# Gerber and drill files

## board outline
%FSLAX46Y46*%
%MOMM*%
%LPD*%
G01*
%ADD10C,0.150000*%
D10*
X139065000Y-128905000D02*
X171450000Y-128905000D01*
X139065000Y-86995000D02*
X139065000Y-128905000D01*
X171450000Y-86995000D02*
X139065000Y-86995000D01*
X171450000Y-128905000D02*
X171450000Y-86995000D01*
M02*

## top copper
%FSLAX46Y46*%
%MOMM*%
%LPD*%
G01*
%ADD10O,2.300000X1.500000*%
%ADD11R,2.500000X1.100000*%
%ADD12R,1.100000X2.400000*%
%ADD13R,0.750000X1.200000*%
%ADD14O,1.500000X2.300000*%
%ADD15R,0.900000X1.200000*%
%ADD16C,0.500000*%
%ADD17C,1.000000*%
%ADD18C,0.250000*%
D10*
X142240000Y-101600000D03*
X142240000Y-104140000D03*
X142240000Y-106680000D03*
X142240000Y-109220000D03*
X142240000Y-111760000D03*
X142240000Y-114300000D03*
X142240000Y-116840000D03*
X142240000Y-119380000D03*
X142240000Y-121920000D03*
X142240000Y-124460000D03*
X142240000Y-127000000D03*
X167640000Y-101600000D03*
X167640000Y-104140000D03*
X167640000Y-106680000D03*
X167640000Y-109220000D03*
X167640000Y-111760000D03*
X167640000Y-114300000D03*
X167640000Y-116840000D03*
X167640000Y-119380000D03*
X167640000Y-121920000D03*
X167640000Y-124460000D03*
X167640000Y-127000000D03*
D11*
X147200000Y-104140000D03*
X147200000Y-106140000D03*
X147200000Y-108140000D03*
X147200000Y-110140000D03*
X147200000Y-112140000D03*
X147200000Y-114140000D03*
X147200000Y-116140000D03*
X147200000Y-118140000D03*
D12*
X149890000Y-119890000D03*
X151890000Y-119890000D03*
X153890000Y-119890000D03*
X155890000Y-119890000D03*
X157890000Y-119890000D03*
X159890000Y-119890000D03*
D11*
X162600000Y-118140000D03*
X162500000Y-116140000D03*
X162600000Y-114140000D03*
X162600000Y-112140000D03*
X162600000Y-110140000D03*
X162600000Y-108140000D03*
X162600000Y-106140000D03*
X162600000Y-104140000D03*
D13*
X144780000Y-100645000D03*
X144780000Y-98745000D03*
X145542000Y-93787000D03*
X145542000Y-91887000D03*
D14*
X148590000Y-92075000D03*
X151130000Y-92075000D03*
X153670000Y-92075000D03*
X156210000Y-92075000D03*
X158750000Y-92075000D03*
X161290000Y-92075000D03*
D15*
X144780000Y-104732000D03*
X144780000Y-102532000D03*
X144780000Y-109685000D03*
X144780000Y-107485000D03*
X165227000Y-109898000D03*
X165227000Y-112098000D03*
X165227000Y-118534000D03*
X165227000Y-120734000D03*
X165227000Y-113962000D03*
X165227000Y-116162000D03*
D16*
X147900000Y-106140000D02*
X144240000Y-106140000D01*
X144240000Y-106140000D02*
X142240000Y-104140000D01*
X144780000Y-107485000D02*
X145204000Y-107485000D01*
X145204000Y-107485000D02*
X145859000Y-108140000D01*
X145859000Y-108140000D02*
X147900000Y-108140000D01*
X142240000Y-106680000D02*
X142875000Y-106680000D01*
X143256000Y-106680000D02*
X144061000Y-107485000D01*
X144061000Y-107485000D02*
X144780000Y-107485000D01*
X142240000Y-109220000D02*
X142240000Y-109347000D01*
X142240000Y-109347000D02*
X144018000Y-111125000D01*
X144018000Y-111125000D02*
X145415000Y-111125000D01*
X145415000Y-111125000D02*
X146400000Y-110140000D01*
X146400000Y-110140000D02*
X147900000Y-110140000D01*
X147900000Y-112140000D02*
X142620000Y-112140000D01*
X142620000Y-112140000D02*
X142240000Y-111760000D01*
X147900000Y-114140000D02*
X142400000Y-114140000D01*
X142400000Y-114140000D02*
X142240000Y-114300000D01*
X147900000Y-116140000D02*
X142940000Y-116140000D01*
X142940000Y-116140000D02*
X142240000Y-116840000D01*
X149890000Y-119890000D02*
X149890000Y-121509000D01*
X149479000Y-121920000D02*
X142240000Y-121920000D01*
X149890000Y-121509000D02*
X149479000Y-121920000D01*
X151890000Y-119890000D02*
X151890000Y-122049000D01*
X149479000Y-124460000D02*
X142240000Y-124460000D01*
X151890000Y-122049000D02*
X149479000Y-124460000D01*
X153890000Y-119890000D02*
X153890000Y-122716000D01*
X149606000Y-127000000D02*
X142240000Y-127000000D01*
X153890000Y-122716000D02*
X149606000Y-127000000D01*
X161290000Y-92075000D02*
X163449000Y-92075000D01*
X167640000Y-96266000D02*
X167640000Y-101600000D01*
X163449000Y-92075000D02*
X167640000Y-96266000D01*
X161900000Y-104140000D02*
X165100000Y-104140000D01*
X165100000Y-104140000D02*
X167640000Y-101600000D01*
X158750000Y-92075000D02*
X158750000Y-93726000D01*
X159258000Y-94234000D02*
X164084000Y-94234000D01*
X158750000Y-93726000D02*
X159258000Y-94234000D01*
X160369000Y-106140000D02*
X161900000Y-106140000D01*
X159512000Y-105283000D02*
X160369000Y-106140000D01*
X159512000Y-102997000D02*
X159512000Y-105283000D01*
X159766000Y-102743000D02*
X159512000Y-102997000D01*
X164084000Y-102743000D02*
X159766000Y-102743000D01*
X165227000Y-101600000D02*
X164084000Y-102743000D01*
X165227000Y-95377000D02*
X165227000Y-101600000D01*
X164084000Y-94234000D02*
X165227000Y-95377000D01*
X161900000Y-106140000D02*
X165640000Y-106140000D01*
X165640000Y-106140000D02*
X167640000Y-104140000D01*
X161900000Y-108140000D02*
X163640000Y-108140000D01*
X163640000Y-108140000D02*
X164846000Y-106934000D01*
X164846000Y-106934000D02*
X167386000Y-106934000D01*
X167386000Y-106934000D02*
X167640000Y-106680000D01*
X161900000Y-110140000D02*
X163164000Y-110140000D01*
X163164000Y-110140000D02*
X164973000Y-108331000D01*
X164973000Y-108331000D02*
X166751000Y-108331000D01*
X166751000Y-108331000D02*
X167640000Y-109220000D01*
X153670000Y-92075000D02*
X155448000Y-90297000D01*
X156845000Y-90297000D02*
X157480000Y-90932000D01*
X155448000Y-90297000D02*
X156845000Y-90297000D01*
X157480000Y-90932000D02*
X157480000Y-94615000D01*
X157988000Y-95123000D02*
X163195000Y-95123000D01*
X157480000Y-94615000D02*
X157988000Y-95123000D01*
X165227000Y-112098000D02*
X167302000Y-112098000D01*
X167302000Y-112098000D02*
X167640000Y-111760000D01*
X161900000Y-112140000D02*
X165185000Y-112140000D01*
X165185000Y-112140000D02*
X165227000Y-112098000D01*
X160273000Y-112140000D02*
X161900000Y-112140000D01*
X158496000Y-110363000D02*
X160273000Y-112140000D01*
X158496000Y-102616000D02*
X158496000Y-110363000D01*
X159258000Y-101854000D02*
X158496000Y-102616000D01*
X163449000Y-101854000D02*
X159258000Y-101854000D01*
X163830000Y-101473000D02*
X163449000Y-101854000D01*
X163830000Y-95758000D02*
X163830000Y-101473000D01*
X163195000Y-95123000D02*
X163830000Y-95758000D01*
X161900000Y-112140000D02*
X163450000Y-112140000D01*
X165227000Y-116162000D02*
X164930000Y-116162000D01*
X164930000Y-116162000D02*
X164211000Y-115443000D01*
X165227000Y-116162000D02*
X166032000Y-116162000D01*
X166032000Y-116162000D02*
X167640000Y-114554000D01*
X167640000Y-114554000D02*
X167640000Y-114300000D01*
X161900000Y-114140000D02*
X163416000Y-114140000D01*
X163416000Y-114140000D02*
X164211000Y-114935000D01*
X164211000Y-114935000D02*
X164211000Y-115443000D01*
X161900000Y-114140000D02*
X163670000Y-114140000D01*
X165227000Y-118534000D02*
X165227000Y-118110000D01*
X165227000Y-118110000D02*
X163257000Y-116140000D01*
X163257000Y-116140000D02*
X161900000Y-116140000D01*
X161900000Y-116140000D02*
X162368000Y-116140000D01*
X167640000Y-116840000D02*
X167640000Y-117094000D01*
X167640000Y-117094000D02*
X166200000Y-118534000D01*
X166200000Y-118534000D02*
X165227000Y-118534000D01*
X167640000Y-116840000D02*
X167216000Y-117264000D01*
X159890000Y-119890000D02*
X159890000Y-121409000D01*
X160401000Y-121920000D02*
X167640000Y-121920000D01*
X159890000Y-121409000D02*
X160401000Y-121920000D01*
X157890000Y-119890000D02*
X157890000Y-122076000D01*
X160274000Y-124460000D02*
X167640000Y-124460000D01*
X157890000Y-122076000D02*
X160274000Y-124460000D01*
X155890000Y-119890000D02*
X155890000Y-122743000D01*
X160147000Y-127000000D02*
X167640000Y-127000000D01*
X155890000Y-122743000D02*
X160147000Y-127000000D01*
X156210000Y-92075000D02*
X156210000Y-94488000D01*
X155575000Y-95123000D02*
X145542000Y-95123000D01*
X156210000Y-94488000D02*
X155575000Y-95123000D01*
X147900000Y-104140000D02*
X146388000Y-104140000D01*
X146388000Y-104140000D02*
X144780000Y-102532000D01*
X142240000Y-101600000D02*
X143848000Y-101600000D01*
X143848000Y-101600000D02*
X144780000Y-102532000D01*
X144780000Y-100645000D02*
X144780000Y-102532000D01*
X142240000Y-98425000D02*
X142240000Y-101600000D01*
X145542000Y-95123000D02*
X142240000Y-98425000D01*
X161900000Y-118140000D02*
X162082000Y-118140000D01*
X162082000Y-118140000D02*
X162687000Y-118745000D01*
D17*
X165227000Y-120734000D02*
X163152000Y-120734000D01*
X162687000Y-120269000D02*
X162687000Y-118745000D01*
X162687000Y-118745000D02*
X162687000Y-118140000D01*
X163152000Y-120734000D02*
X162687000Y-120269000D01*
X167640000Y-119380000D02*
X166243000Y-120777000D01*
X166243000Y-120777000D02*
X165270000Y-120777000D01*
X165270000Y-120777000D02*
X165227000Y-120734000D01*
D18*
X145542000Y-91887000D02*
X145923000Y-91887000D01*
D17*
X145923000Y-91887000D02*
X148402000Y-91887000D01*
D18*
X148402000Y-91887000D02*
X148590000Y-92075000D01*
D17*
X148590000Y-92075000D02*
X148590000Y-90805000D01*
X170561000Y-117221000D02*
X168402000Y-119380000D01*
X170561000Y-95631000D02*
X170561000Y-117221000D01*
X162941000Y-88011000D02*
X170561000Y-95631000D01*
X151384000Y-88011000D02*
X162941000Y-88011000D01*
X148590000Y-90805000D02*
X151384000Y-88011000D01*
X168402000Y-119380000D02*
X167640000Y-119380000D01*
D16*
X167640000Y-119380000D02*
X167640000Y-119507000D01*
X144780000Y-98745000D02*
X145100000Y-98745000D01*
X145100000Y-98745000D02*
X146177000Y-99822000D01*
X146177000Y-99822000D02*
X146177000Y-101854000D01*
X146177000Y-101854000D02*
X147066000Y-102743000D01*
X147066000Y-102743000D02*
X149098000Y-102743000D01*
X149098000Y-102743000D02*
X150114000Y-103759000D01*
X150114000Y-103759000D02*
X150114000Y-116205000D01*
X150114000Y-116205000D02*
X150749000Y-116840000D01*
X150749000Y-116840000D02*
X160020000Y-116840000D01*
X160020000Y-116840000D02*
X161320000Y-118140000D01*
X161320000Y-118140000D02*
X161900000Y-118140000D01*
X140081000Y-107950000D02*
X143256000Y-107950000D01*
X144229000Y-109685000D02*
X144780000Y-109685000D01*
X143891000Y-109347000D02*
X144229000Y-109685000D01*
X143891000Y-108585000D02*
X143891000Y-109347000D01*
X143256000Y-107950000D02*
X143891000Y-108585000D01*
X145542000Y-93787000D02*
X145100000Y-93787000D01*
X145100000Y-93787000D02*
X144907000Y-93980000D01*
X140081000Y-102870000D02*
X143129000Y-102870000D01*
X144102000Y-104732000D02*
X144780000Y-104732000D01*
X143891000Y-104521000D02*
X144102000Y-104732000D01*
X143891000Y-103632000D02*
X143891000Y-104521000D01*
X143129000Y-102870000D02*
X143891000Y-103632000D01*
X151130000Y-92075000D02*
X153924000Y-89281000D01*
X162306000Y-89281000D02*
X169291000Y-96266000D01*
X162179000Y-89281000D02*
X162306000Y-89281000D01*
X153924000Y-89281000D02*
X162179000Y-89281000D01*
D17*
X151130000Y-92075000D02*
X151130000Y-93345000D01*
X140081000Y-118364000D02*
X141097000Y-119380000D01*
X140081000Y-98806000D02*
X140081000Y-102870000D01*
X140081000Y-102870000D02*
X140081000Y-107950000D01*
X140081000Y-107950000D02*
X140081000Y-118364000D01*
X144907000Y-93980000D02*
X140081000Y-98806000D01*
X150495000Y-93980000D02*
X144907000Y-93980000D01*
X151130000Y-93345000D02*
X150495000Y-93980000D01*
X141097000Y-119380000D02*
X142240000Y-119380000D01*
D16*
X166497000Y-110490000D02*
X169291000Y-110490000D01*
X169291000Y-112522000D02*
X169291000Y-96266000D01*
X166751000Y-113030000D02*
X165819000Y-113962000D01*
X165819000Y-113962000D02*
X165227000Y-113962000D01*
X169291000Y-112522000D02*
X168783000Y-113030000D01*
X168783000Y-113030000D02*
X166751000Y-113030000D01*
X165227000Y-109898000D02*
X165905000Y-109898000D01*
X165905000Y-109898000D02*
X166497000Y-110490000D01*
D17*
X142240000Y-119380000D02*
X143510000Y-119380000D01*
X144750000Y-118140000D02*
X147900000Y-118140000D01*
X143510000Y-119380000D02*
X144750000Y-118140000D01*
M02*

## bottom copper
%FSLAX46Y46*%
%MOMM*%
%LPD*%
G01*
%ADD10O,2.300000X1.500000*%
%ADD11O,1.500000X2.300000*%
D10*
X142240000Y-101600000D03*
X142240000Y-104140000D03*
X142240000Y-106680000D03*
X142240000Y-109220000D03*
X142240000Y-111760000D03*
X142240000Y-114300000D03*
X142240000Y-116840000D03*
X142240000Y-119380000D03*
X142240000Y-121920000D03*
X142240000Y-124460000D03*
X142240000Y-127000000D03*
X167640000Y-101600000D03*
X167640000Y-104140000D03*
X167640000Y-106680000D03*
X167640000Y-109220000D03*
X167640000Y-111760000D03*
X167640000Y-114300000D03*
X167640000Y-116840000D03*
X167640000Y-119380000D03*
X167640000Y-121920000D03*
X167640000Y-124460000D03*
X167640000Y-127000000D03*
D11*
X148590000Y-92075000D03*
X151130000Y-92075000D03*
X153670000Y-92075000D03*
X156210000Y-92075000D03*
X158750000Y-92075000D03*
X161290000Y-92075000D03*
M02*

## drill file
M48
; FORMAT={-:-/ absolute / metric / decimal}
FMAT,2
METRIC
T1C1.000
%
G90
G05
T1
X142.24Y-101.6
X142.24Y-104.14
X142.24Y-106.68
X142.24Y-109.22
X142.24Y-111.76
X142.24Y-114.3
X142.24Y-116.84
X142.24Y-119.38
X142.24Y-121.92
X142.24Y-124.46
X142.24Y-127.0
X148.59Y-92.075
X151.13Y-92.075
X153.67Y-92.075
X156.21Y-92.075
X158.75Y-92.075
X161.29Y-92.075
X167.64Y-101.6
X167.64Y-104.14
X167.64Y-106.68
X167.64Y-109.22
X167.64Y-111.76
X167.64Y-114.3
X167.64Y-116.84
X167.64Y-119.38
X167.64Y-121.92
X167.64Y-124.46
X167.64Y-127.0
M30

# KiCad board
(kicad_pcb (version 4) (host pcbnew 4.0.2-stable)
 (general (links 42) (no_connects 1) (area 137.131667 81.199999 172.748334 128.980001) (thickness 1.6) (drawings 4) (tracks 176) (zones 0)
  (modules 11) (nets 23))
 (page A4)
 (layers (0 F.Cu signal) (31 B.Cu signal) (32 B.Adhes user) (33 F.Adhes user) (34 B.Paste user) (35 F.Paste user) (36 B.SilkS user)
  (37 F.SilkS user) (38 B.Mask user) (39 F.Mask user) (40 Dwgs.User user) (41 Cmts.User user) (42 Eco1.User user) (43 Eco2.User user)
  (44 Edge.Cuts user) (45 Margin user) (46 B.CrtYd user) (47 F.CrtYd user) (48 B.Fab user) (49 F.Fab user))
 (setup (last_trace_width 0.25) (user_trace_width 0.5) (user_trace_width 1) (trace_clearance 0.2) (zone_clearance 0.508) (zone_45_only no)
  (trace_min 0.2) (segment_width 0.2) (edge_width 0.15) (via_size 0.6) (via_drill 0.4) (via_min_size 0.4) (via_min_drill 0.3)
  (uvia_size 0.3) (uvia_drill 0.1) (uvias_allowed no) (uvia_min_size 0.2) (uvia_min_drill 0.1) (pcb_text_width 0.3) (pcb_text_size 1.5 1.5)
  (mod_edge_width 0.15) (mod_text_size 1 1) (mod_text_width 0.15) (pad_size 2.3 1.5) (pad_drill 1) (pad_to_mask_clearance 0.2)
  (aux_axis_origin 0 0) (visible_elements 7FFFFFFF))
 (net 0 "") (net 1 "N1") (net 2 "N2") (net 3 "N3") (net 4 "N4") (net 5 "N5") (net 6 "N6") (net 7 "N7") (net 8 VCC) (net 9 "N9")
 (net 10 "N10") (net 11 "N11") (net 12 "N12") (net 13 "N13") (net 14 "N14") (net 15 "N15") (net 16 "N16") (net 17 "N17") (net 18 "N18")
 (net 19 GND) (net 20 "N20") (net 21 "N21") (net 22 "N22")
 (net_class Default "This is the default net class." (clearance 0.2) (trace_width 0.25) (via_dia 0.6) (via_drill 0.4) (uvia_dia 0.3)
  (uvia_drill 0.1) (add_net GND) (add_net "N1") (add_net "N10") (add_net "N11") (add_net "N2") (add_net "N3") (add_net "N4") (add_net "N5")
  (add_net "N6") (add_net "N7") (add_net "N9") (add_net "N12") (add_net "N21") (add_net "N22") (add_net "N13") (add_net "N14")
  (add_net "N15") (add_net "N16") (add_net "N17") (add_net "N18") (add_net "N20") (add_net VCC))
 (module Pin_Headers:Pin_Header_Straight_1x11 (layer F.Cu) (at 142.24 101.6)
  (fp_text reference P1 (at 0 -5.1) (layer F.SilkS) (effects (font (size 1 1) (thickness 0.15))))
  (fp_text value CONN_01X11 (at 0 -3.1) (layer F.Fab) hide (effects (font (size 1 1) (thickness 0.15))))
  (pad 1 thru_hole oval (at 0 0) (size 2.3 1.5) (drill 1) (layers *.Cu *.Mask) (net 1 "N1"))
  (pad 2 thru_hole oval (at 0 2.54) (size 2.3 1.5) (drill 1) (layers *.Cu *.Mask) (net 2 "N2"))
  (pad 3 thru_hole oval (at 0 5.08) (size 2.3 1.5) (drill 1) (layers *.Cu *.Mask) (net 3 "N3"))
  (pad 4 thru_hole oval (at 0 7.62) (size 2.3 1.5) (drill 1) (layers *.Cu *.Mask) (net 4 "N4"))
  (pad 5 thru_hole oval (at 0 10.16) (size 2.3 1.5) (drill 1) (layers *.Cu *.Mask) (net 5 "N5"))
  (pad 6 thru_hole oval (at 0 12.7) (size 2.3 1.5) (drill 1) (layers *.Cu *.Mask) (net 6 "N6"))
  (pad 7 thru_hole oval (at 0 15.24) (size 2.3 1.5) (drill 1) (layers *.Cu *.Mask) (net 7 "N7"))
  (pad 8 thru_hole oval (at 0 17.78) (size 2.3 1.5) (drill 1) (layers *.Cu *.Mask) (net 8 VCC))
  (pad 9 thru_hole oval (at 0 20.32) (size 2.3 1.5) (drill 1) (layers *.Cu *.Mask) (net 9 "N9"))
  (pad 10 thru_hole oval (at 0 22.86) (size 2.3 1.5) (drill 1) (layers *.Cu *.Mask) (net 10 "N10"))
  (pad 11 thru_hole oval (at 0 25.4) (size 2.3 1.5) (drill 1) (layers *.Cu *.Mask) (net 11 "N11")))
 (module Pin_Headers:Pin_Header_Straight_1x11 (layer F.Cu) (at 167.64 101.6)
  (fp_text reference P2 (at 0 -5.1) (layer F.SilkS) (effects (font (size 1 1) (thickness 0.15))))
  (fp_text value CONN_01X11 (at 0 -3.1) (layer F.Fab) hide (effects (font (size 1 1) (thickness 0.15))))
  (pad 1 thru_hole oval (at 0 0) (size 2.3 1.5) (drill 1) (layers *.Cu *.Mask) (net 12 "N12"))
  (pad 2 thru_hole oval (at 0 2.54) (size 2.3 1.5) (drill 1) (layers *.Cu *.Mask) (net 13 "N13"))
  (pad 3 thru_hole oval (at 0 5.08) (size 2.3 1.5) (drill 1) (layers *.Cu *.Mask) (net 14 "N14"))
  (pad 4 thru_hole oval (at 0 7.62) (size 2.3 1.5) (drill 1) (layers *.Cu *.Mask) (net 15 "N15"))
  (pad 5 thru_hole oval (at 0 10.16) (size 2.3 1.5) (drill 1) (layers *.Cu *.Mask) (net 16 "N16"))
  (pad 6 thru_hole oval (at 0 12.7) (size 2.3 1.5) (drill 1) (layers *.Cu *.Mask) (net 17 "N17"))
  (pad 7 thru_hole oval (at 0 15.24) (size 2.3 1.5) (drill 1) (layers *.Cu *.Mask) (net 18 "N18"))
  (pad 8 thru_hole oval (at 0 17.78) (size 2.3 1.5) (drill 1) (layers *.Cu *.Mask) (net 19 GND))
  (pad 9 thru_hole oval (at 0 20.32) (size 2.3 1.5) (drill 1) (layers *.Cu *.Mask) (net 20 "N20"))
  (pad 10 thru_hole oval (at 0 22.86) (size 2.3 1.5) (drill 1) (layers *.Cu *.Mask) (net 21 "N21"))
  (pad 11 thru_hole oval (at 0 25.4) (size 2.3 1.5) (drill 1) (layers *.Cu *.Mask) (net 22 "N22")))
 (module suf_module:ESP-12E (layer F.Cu) (at 147.9 104.14)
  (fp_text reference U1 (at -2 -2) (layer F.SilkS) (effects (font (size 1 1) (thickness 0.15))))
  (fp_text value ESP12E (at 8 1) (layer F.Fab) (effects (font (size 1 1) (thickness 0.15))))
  (pad 1 smd rect (at 0 0) (size 2.5 1.1) (drill (offset -0.7 0)) (layers F.Cu F.Paste F.Mask) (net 1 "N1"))
  (pad 2 smd rect (at 0 2) (size 2.5 1.1) (drill (offset -0.7 0)) (layers F.Cu F.Paste F.Mask) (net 2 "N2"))
  (pad 3 smd rect (at 0 4) (size 2.5 1.1) (drill (offset -0.7 0)) (layers F.Cu F.Paste F.Mask) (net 3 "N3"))
  (pad 4 smd rect (at 0 6) (size 2.5 1.1) (drill (offset -0.7 0)) (layers F.Cu F.Paste F.Mask) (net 4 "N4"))
  (pad 5 smd rect (at 0 8) (size 2.5 1.1) (drill (offset -0.7 0)) (layers F.Cu F.Paste F.Mask) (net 5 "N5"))
  (pad 6 smd rect (at 0 10) (size 2.5 1.1) (drill (offset -0.7 0)) (layers F.Cu F.Paste F.Mask) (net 6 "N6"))
  (pad 7 smd rect (at 0 12) (size 2.5 1.1) (drill (offset -0.7 0)) (layers F.Cu F.Paste F.Mask) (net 7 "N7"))
  (pad 8 smd rect (at 0 14) (size 2.5 1.1) (drill (offset -0.7 0)) (layers F.Cu F.Paste F.Mask) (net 8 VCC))
  (pad 17 smd rect (at 1.99 15.75 90) (size 2.4 1.1) (layers F.Cu F.Paste F.Mask) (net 9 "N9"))
  (pad 18 smd rect (at 3.99 15.75 90) (size 2.4 1.1) (layers F.Cu F.Paste F.Mask) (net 10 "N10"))
  (pad 19 smd rect (at 5.99 15.75 90) (size 2.4 1.1) (layers F.Cu F.Paste F.Mask) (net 11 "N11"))
  (pad 20 smd rect (at 7.99 15.75 90) (size 2.4 1.1) (layers F.Cu F.Paste F.Mask) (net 22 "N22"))
  (pad 21 smd rect (at 9.99 15.75 90) (size 2.4 1.1) (layers F.Cu F.Paste F.Mask) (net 21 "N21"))
  (pad 22 smd rect (at 11.99 15.75 90) (size 2.4 1.1) (layers F.Cu F.Paste F.Mask) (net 20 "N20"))
  (pad 9 smd rect (at 14 14) (size 2.5 1.1) (drill (offset 0.7 0)) (layers F.Cu F.Paste F.Mask) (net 19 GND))
  (pad 10 smd rect (at 14 12) (size 2.5 1.1) (drill (offset 0.6 0)) (layers F.Cu F.Paste F.Mask) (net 18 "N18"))
  (pad 11 smd rect (at 14 10) (size 2.5 1.1) (drill (offset 0.7 0)) (layers F.Cu F.Paste F.Mask) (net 17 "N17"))
  (pad 12 smd rect (at 14 8) (size 2.5 1.1) (drill (offset 0.7 0)) (layers F.Cu F.Paste F.Mask) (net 16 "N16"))
  (pad 13 smd rect (at 14 6) (size 2.5 1.1) (drill (offset 0.7 0)) (layers F.Cu F.Paste F.Mask) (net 15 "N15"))
  (pad 14 smd rect (at 14 4) (size 2.5 1.1) (drill (offset 0.7 0)) (layers F.Cu F.Paste F.Mask) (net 14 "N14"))
  (pad 15 smd rect (at 14 2) (size 2.5 1.1) (drill (offset 0.7 0)) (layers F.Cu F.Paste F.Mask) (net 13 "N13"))
  (pad 16 smd rect (at 14 0) (size 2.5 1.1) (drill (offset 0.7 0)) (layers F.Cu F.Paste F.Mask) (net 12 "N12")))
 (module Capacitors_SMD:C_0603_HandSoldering (layer F.Cu) (at 144.78 99.695 90)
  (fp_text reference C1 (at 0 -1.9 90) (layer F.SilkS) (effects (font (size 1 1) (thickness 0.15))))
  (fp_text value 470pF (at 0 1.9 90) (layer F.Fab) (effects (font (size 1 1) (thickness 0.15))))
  (pad 1 smd rect (at -0.95 0 90) (size 1.2 0.75) (layers F.Cu F.Paste F.Mask) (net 1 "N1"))
  (pad 2 smd rect (at 0.95 0 90) (size 1.2 0.75) (layers F.Cu F.Paste F.Mask) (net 19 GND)))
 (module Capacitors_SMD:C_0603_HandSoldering (layer F.Cu) (at 145.542 92.837 90)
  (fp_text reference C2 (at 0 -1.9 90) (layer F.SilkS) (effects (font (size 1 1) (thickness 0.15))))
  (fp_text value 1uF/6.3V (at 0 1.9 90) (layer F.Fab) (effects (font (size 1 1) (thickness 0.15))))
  (pad 1 smd rect (at -0.95 0 90) (size 1.2 0.75) (layers F.Cu F.Paste F.Mask) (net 8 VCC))
  (pad 2 smd rect (at 0.95 0 90) (size 1.2 0.75) (layers F.Cu F.Paste F.Mask) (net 19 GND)))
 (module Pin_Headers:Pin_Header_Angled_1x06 (layer F.Cu) (at 148.59 92.075 90)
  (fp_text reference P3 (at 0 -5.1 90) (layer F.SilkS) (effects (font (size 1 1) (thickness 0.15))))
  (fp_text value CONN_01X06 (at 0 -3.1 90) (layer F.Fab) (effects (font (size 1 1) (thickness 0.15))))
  (pad 1 thru_hole oval (at 0 0 90) (size 2.3 1.5) (drill 1) (layers *.Cu *.Mask) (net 19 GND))
  (pad 2 thru_hole oval (at 0 2.54 90) (size 2.3 1.5) (drill 1) (layers *.Cu *.Mask) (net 8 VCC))
  (pad 3 thru_hole oval (at 0 5.08 90) (size 2.3 1.5) (drill 1) (layers *.Cu *.Mask) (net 16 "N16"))
  (pad 4 thru_hole oval (at 0 7.62 90) (size 2.3 1.5) (drill 1) (layers *.Cu *.Mask) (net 1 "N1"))
  (pad 5 thru_hole oval (at 0 10.16 90) (size 2.3 1.5) (drill 1) (layers *.Cu *.Mask) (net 13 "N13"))
  (pad 6 thru_hole oval (at 0 12.7 90) (size 2.3 1.5) (drill 1) (layers *.Cu *.Mask) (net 12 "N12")))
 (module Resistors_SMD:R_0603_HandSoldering (layer F.Cu) (at 144.78 103.632 90)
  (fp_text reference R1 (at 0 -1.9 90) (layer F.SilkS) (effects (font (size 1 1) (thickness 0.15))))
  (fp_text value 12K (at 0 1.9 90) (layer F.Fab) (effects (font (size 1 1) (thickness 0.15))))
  (pad 1 smd rect (at -1.1 0 90) (size 1.2 0.9) (layers F.Cu F.Paste F.Mask) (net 8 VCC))
  (pad 2 smd rect (at 1.1 0 90) (size 1.2 0.9) (layers F.Cu F.Paste F.Mask) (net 1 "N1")))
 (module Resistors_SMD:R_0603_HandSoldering (layer F.Cu) (at 144.78 108.585 90)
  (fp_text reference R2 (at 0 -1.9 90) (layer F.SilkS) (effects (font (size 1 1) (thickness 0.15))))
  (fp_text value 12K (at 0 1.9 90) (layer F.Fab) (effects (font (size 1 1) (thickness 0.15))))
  (pad 1 smd rect (at -1.1 0 90) (size 1.2 0.9) (layers F.Cu F.Paste F.Mask) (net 8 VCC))
  (pad 2 smd rect (at 1.1 0 90) (size 1.2 0.9) (layers F.Cu F.Paste F.Mask) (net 3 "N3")))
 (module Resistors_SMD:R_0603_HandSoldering (layer F.Cu) (at 165.227 110.998 270)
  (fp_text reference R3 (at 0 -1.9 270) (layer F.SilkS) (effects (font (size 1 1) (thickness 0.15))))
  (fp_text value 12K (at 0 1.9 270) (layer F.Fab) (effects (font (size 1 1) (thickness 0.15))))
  (pad 1 smd rect (at -1.1 0 270) (size 1.2 0.9) (layers F.Cu F.Paste F.Mask) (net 8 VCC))
  (pad 2 smd rect (at 1.1 0 270) (size 1.2 0.9) (layers F.Cu F.Paste F.Mask) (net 16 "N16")))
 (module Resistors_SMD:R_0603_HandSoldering (layer F.Cu) (at 165.227 119.634 270)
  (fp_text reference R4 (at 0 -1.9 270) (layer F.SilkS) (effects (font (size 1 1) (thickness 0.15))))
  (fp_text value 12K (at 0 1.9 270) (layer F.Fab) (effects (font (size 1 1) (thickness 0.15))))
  (pad 1 smd rect (at -1.1 0 270) (size 1.2 0.9) (layers F.Cu F.Paste F.Mask) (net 18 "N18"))
  (pad 2 smd rect (at 1.1 0 270) (size 1.2 0.9) (layers F.Cu F.Paste F.Mask) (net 19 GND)))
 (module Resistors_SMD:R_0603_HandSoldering (layer F.Cu) (at 165.227 115.062 270)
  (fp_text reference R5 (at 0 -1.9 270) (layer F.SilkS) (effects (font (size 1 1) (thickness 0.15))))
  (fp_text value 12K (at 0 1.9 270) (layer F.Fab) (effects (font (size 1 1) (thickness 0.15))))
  (pad 1 smd rect (at -1.1 0 270) (size 1.2 0.9) (layers F.Cu F.Paste F.Mask) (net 8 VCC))
  (pad 2 smd rect (at 1.1 0 270) (size 1.2 0.9) (layers F.Cu F.Paste F.Mask) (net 17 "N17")))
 (gr_line (start 139.065 128.905) (end 171.45 128.905) (angle 90) (layer Edge.Cuts) (width 0.15))
 (gr_line (start 139.065 86.995) (end 139.065 128.905) (angle 90) (layer Edge.Cuts) (width 0.15))
 (gr_line (start 171.45 86.995) (end 139.065 86.995) (angle 90) (layer Edge.Cuts) (width 0.15))
 (gr_line (start 171.45 128.905) (end 171.45 86.995) (angle 90) (layer Edge.Cuts) (width 0.15))
 (segment (start 147.9 106.14) (end 144.24 106.14) (width 0.5) (layer F.Cu) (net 2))
 (segment (start 144.24 106.14) (end 142.24 104.14) (width 0.5) (layer F.Cu) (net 2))
 (segment (start 144.78 107.485) (end 145.204 107.485) (width 0.5) (layer F.Cu) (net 3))
 (segment (start 145.204 107.485) (end 145.859 108.14) (width 0.5) (layer F.Cu) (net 3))
 (segment (start 145.859 108.14) (end 147.9 108.14) (width 0.5) (layer F.Cu) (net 3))
 (segment (start 142.24 106.68) (end 142.875 106.68) (width 0.5) (layer F.Cu) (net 3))
 (segment (start 143.256 106.68) (end 144.061 107.485) (width 0.5) (layer F.Cu) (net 3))
 (segment (start 144.061 107.485) (end 144.78 107.485) (width 0.5) (layer F.Cu) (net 3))
 (segment (start 142.24 109.22) (end 142.24 109.347) (width 0.5) (layer F.Cu) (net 4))
 (segment (start 142.24 109.347) (end 144.018 111.125) (width 0.5) (layer F.Cu) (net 4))
 (segment (start 144.018 111.125) (end 145.415 111.125) (width 0.5) (layer F.Cu) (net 4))
 (segment (start 145.415 111.125) (end 146.4 110.14) (width 0.5) (layer F.Cu) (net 4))
 (segment (start 146.4 110.14) (end 147.9 110.14) (width 0.5) (layer F.Cu) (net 4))
 (segment (start 147.9 112.14) (end 142.62 112.14) (width 0.5) (layer F.Cu) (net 5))
 (segment (start 142.62 112.14) (end 142.24 111.76) (width 0.5) (layer F.Cu) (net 5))
 (segment (start 147.9 114.14) (end 142.4 114.14) (width 0.5) (layer F.Cu) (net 6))
 (segment (start 142.4 114.14) (end 142.24 114.3) (width 0.5) (layer F.Cu) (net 6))
 (segment (start 147.9 116.14) (end 142.94 116.14) (width 0.5) (layer F.Cu) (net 7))
 (segment (start 142.94 116.14) (end 142.24 116.84) (width 0.5) (layer F.Cu) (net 7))
 (segment (start 149.89 119.89) (end 149.89 121.509) (width 0.5) (layer F.Cu) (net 9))
 (segment (start 149.479 121.92) (end 142.24 121.92) (width 0.5) (layer F.Cu) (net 9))
 (segment (start 149.89 121.509) (end 149.479 121.92) (width 0.5) (layer F.Cu) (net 9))
 (segment (start 151.89 119.89) (end 151.89 122.049) (width 0.5) (layer F.Cu) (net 10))
 (segment (start 149.479 124.46) (end 142.24 124.46) (width 0.5) (layer F.Cu) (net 10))
 (segment (start 151.89 122.049) (end 149.479 124.46) (width 0.5) (layer F.Cu) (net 10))
 (segment (start 153.89 119.89) (end 153.89 122.716) (width 0.5) (layer F.Cu) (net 11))
 (segment (start 149.606 127) (end 142.24 127) (width 0.5) (layer F.Cu) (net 11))
 (segment (start 153.89 122.716) (end 149.606 127) (width 0.5) (layer F.Cu) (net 11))
 (segment (start 161.29 92.075) (end 163.449 92.075) (width 0.5) (layer F.Cu) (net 12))
 (segment (start 167.64 96.266) (end 167.64 101.6) (width 0.5) (layer F.Cu) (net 12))
 (segment (start 163.449 92.075) (end 167.64 96.266) (width 0.5) (layer F.Cu) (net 12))
 (segment (start 161.9 104.14) (end 165.1 104.14) (width 0.5) (layer F.Cu) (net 12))
 (segment (start 165.1 104.14) (end 167.64 101.6) (width 0.5) (layer F.Cu) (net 12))
 (segment (start 158.75 92.075) (end 158.75 93.726) (width 0.5) (layer F.Cu) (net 13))
 (segment (start 159.258 94.234) (end 164.084 94.234) (width 0.5) (layer F.Cu) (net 13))
 (segment (start 158.75 93.726) (end 159.258 94.234) (width 0.5) (layer F.Cu) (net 13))
 (segment (start 160.369 106.14) (end 161.9 106.14) (width 0.5) (layer F.Cu) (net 13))
 (segment (start 159.512 105.283) (end 160.369 106.14) (width 0.5) (layer F.Cu) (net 13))
 (segment (start 159.512 102.997) (end 159.512 105.283) (width 0.5) (layer F.Cu) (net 13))
 (segment (start 159.766 102.743) (end 159.512 102.997) (width 0.5) (layer F.Cu) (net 13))
 (segment (start 164.084 102.743) (end 159.766 102.743) (width 0.5) (layer F.Cu) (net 13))
 (segment (start 165.227 101.6) (end 164.084 102.743) (width 0.5) (layer F.Cu) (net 13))
 (segment (start 165.227 95.377) (end 165.227 101.6) (width 0.5) (layer F.Cu) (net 13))
 (segment (start 164.084 94.234) (end 165.227 95.377) (width 0.5) (layer F.Cu) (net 13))
 (segment (start 161.9 106.14) (end 165.64 106.14) (width 0.5) (layer F.Cu) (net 13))
 (segment (start 165.64 106.14) (end 167.64 104.14) (width 0.5) (layer F.Cu) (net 13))
 (segment (start 161.9 108.14) (end 163.64 108.14) (width 0.5) (layer F.Cu) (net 14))
 (segment (start 163.64 108.14) (end 164.846 106.934) (width 0.5) (layer F.Cu) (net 14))
 (segment (start 164.846 106.934) (end 167.386 106.934) (width 0.5) (layer F.Cu) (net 14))
 (segment (start 167.386 106.934) (end 167.64 106.68) (width 0.5) (layer F.Cu) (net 14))
 (segment (start 161.9 110.14) (end 163.164 110.14) (width 0.5) (layer F.Cu) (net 15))
 (segment (start 163.164 110.14) (end 164.973 108.331) (width 0.5) (layer F.Cu) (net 15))
 (segment (start 164.973 108.331) (end 166.751 108.331) (width 0.5) (layer F.Cu) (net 15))
 (segment (start 166.751 108.331) (end 167.64 109.22) (width 0.5) (layer F.Cu) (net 15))
 (segment (start 153.67 92.075) (end 155.448 90.297) (width 0.5) (layer F.Cu) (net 16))
 (segment (start 156.845 90.297) (end 157.48 90.932) (width 0.5) (layer F.Cu) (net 16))
 (segment (start 155.448 90.297) (end 156.845 90.297) (width 0.5) (layer F.Cu) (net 16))
 (segment (start 157.48 90.932) (end 157.48 94.615) (width 0.5) (layer F.Cu) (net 16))
 (segment (start 157.988 95.123) (end 163.195 95.123) (width 0.5) (layer F.Cu) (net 16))
 (segment (start 157.48 94.615) (end 157.988 95.123) (width 0.5) (layer F.Cu) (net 16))
 (segment (start 165.227 112.098) (end 167.302 112.098) (width 0.5) (layer F.Cu) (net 16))
 (segment (start 167.302 112.098) (end 167.64 111.76) (width 0.5) (layer F.Cu) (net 16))
 (segment (start 161.9 112.14) (end 165.185 112.14) (width 0.5) (layer F.Cu) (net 16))
 (segment (start 165.185 112.14) (end 165.227 112.098) (width 0.5) (layer F.Cu) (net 16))
 (segment (start 160.273 112.14) (end 161.9 112.14) (width 0.5) (layer F.Cu) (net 16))
 (segment (start 158.496 110.363) (end 160.273 112.14) (width 0.5) (layer F.Cu) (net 16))
 (segment (start 158.496 102.616) (end 158.496 110.363) (width 0.5) (layer F.Cu) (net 16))
 (segment (start 159.258 101.854) (end 158.496 102.616) (width 0.5) (layer F.Cu) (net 16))
 (segment (start 163.449 101.854) (end 159.258 101.854) (width 0.5) (layer F.Cu) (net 16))
 (segment (start 163.83 101.473) (end 163.449 101.854) (width 0.5) (layer F.Cu) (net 16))
 (segment (start 163.83 95.758) (end 163.83 101.473) (width 0.5) (layer F.Cu) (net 16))
 (segment (start 163.195 95.123) (end 163.83 95.758) (width 0.5) (layer F.Cu) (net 16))
 (segment (start 161.9 112.14) (end 163.45 112.14) (width 0.5) (layer F.Cu) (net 16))
 (segment (start 165.227 116.162) (end 164.93 116.162) (width 0.5) (layer F.Cu) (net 17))
 (segment (start 164.93 116.162) (end 164.211 115.443) (width 0.5) (layer F.Cu) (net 17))
 (segment (start 165.227 116.162) (end 166.032 116.162) (width 0.5) (layer F.Cu) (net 17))
 (segment (start 166.032 116.162) (end 167.64 114.554) (width 0.5) (layer F.Cu) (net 17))
 (segment (start 167.64 114.554) (end 167.64 114.3) (width 0.5) (layer F.Cu) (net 17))
 (segment (start 161.9 114.14) (end 163.416 114.14) (width 0.5) (layer F.Cu) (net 17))
 (segment (start 163.416 114.14) (end 164.211 114.935) (width 0.5) (layer F.Cu) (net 17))
 (segment (start 164.211 114.935) (end 164.211 115.443) (width 0.5) (layer F.Cu) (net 17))
 (segment (start 161.9 114.14) (end 163.67 114.14) (width 0.5) (layer F.Cu) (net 17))
 (segment (start 165.227 118.534) (end 165.227 118.11) (width 0.5) (layer F.Cu) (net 18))
 (segment (start 165.227 118.11) (end 163.257 116.14) (width 0.5) (layer F.Cu) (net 18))
 (segment (start 163.257 116.14) (end 161.9 116.14) (width 0.5) (layer F.Cu) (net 18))
 (segment (start 161.9 116.14) (end 162.368 116.14) (width 0.5) (layer F.Cu) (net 18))
 (segment (start 167.64 116.84) (end 167.64 117.094) (width 0.5) (layer F.Cu) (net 18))
 (segment (start 167.64 117.094) (end 166.2 118.534) (width 0.5) (layer F.Cu) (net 18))
 (segment (start 166.2 118.534) (end 165.227 118.534) (width 0.5) (layer F.Cu) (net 18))
 (segment (start 167.64 116.84) (end 167.216 117.264) (width 0.5) (layer F.Cu) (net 18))
 (segment (start 159.89 119.89) (end 159.89 121.409) (width 0.5) (layer F.Cu) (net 20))
 (segment (start 160.401 121.92) (end 167.64 121.92) (width 0.5) (layer F.Cu) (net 20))
 (segment (start 159.89 121.409) (end 160.401 121.92) (width 0.5) (layer F.Cu) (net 20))
 (segment (start 157.89 119.89) (end 157.89 122.076) (width 0.5) (layer F.Cu) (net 21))
 (segment (start 160.274 124.46) (end 167.64 124.46) (width 0.5) (layer F.Cu) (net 21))
 (segment (start 157.89 122.076) (end 160.274 124.46) (width 0.5) (layer F.Cu) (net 21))
 (segment (start 155.89 119.89) (end 155.89 122.743) (width 0.5) (layer F.Cu) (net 22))
 (segment (start 160.147 127) (end 167.64 127) (width 0.5) (layer F.Cu) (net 22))
 (segment (start 155.89 122.743) (end 160.147 127) (width 0.5) (layer F.Cu) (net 22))
 (segment (start 156.21 92.075) (end 156.21 94.488) (width 0.5) (layer F.Cu) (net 1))
 (segment (start 155.575 95.123) (end 145.542 95.123) (width 0.5) (layer F.Cu) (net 1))
 (segment (start 156.21 94.488) (end 155.575 95.123) (width 0.5) (layer F.Cu) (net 1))
 (segment (start 147.9 104.14) (end 146.388 104.14) (width 0.5) (layer F.Cu) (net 1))
 (segment (start 146.388 104.14) (end 144.78 102.532) (width 0.5) (layer F.Cu) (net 1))
 (segment (start 142.24 101.6) (end 143.848 101.6) (width 0.5) (layer F.Cu) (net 1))
 (segment (start 143.848 101.6) (end 144.78 102.532) (width 0.5) (layer F.Cu) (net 1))
 (segment (start 144.78 100.645) (end 144.78 102.532) (width 0.5) (layer F.Cu) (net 1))
 (segment (start 142.24 98.425) (end 142.24 101.6) (width 0.5) (layer F.Cu) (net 1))
 (segment (start 145.542 95.123) (end 142.24 98.425) (width 0.5) (layer F.Cu) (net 1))
 (segment (start 161.9 118.14) (end 162.082 118.14) (width 0.5) (layer F.Cu) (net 19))
 (segment (start 162.082 118.14) (end 162.687 118.745) (width 0.5) (layer F.Cu) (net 19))
 (segment (start 165.227 120.734) (end 163.152 120.734) (width 1) (layer F.Cu) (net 19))
 (segment (start 162.687 120.269) (end 162.687 118.745) (width 1) (layer F.Cu) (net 19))
 (segment (start 162.687 118.745) (end 162.687 118.14) (width 1) (layer F.Cu) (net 19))
 (segment (start 163.152 120.734) (end 162.687 120.269) (width 1) (layer F.Cu) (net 19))
 (segment (start 167.64 119.38) (end 166.243 120.777) (width 1) (layer F.Cu) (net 19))
 (segment (start 166.243 120.777) (end 165.27 120.777) (width 1) (layer F.Cu) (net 19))
 (segment (start 165.27 120.777) (end 165.227 120.734) (width 1) (layer F.Cu) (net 19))
 (segment (start 145.542 91.887) (end 145.923 91.887) (width 0.25) (layer F.Cu) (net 19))
 (segment (start 145.923 91.887) (end 148.402 91.887) (width 1) (layer F.Cu) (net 19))
 (segment (start 148.402 91.887) (end 148.59 92.075) (width 0.25) (layer F.Cu) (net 19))
 (segment (start 148.59 92.075) (end 148.59 90.805) (width 1) (layer F.Cu) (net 19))
 (segment (start 170.561 117.221) (end 168.402 119.38) (width 1) (layer F.Cu) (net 19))
 (segment (start 170.561 95.631) (end 170.561 117.221) (width 1) (layer F.Cu) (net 19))
 (segment (start 162.941 88.011) (end 170.561 95.631) (width 1) (layer F.Cu) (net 19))
 (segment (start 151.384 88.011) (end 162.941 88.011) (width 1) (layer F.Cu) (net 19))
 (segment (start 148.59 90.805) (end 151.384 88.011) (width 1) (layer F.Cu) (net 19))
 (segment (start 168.402 119.38) (end 167.64 119.38) (width 1) (layer F.Cu) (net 19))
 (segment (start 167.64 119.38) (end 167.64 119.507) (width 0.5) (layer F.Cu) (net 19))
 (segment (start 144.78 98.745) (end 145.1 98.745) (width 0.5) (layer F.Cu) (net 19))
 (segment (start 145.1 98.745) (end 146.177 99.822) (width 0.5) (layer F.Cu) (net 19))
 (segment (start 146.177 99.822) (end 146.177 101.854) (width 0.5) (layer F.Cu) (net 19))
 (segment (start 146.177 101.854) (end 147.066 102.743) (width 0.5) (layer F.Cu) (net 19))
 (segment (start 147.066 102.743) (end 149.098 102.743) (width 0.5) (layer F.Cu) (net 19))
 (segment (start 149.098 102.743) (end 150.114 103.759) (width 0.5) (layer F.Cu) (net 19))
 (segment (start 150.114 103.759) (end 150.114 116.205) (width 0.5) (layer F.Cu) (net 19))
 (segment (start 150.114 116.205) (end 150.749 116.84) (width 0.5) (layer F.Cu) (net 19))
 (segment (start 150.749 116.84) (end 160.02 116.84) (width 0.5) (layer F.Cu) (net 19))
 (segment (start 160.02 116.84) (end 161.32 118.14) (width 0.5) (layer F.Cu) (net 19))
 (segment (start 161.32 118.14) (end 161.9 118.14) (width 0.5) (layer F.Cu) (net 19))
 (segment (start 140.081 107.95) (end 143.256 107.95) (width 0.5) (layer F.Cu) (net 8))
 (segment (start 144.229 109.685) (end 144.78 109.685) (width 0.5) (layer F.Cu) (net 8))
 (segment (start 143.891 109.347) (end 144.229 109.685) (width 0.5) (layer F.Cu) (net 8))
 (segment (start 143.891 108.585) (end 143.891 109.347) (width 0.5) (layer F.Cu) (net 8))
 (segment (start 143.256 107.95) (end 143.891 108.585) (width 0.5) (layer F.Cu) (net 8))
 (segment (start 145.542 93.787) (end 145.1 93.787) (width 0.5) (layer F.Cu) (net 8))
 (segment (start 145.1 93.787) (end 144.907 93.98) (width 0.5) (layer F.Cu) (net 8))
 (segment (start 140.081 102.87) (end 143.129 102.87) (width 0.5) (layer F.Cu) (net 8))
 (segment (start 144.102 104.732) (end 144.78 104.732) (width 0.5) (layer F.Cu) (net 8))
 (segment (start 143.891 104.521) (end 144.102 104.732) (width 0.5) (layer F.Cu) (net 8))
 (segment (start 143.891 103.632) (end 143.891 104.521) (width 0.5) (layer F.Cu) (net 8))
 (segment (start 143.129 102.87) (end 143.891 103.632) (width 0.5) (layer F.Cu) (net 8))
 (segment (start 151.13 92.075) (end 153.924 89.281) (width 0.5) (layer F.Cu) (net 8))
 (segment (start 162.306 89.281) (end 169.291 96.266) (width 0.5) (layer F.Cu) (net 8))
 (segment (start 162.179 89.281) (end 162.306 89.281) (width 0.5) (layer F.Cu) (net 8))
 (segment (start 153.924 89.281) (end 162.179 89.281) (width 0.5) (layer F.Cu) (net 8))
 (segment (start 151.13 92.075) (end 151.13 93.345) (width 1) (layer F.Cu) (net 8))
 (segment (start 140.081 118.364) (end 141.097 119.38) (width 1) (layer F.Cu) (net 8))
 (segment (start 140.081 98.806) (end 140.081 102.87) (width 1) (layer F.Cu) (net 8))
 (segment (start 140.081 102.87) (end 140.081 107.95) (width 1) (layer F.Cu) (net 8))
 (segment (start 140.081 107.95) (end 140.081 118.364) (width 1) (layer F.Cu) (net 8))
 (segment (start 144.907 93.98) (end 140.081 98.806) (width 1) (layer F.Cu) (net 8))
 (segment (start 150.495 93.98) (end 144.907 93.98) (width 1) (layer F.Cu) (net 8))
 (segment (start 151.13 93.345) (end 150.495 93.98) (width 1) (layer F.Cu) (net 8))
 (segment (start 141.097 119.38) (end 142.24 119.38) (width 1) (layer F.Cu) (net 8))
 (segment (start 166.497 110.49) (end 169.291 110.49) (width 0.5) (layer F.Cu) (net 8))
 (segment (start 169.291 112.522) (end 169.291 96.266) (width 0.5) (layer F.Cu) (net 8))
 (segment (start 166.751 113.03) (end 165.819 113.962) (width 0.5) (layer F.Cu) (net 8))
 (segment (start 165.819 113.962) (end 165.227 113.962) (width 0.5) (layer F.Cu) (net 8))
 (segment (start 169.291 112.522) (end 168.783 113.03) (width 0.5) (layer F.Cu) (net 8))
 (segment (start 168.783 113.03) (end 166.751 113.03) (width 0.5) (layer F.Cu) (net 8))
 (segment (start 165.227 109.898) (end 165.905 109.898) (width 0.5) (layer F.Cu) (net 8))
 (segment (start 165.905 109.898) (end 166.497 110.49) (width 0.5) (layer F.Cu) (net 8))
 (segment (start 142.24 119.38) (end 143.51 119.38) (width 1) (layer F.Cu) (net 8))
 (segment (start 144.75 118.14) (end 147.9 118.14) (width 1) (layer F.Cu) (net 8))
 (segment (start 143.51 119.38) (end 144.75 118.14) (width 1) (layer F.Cu) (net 8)))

